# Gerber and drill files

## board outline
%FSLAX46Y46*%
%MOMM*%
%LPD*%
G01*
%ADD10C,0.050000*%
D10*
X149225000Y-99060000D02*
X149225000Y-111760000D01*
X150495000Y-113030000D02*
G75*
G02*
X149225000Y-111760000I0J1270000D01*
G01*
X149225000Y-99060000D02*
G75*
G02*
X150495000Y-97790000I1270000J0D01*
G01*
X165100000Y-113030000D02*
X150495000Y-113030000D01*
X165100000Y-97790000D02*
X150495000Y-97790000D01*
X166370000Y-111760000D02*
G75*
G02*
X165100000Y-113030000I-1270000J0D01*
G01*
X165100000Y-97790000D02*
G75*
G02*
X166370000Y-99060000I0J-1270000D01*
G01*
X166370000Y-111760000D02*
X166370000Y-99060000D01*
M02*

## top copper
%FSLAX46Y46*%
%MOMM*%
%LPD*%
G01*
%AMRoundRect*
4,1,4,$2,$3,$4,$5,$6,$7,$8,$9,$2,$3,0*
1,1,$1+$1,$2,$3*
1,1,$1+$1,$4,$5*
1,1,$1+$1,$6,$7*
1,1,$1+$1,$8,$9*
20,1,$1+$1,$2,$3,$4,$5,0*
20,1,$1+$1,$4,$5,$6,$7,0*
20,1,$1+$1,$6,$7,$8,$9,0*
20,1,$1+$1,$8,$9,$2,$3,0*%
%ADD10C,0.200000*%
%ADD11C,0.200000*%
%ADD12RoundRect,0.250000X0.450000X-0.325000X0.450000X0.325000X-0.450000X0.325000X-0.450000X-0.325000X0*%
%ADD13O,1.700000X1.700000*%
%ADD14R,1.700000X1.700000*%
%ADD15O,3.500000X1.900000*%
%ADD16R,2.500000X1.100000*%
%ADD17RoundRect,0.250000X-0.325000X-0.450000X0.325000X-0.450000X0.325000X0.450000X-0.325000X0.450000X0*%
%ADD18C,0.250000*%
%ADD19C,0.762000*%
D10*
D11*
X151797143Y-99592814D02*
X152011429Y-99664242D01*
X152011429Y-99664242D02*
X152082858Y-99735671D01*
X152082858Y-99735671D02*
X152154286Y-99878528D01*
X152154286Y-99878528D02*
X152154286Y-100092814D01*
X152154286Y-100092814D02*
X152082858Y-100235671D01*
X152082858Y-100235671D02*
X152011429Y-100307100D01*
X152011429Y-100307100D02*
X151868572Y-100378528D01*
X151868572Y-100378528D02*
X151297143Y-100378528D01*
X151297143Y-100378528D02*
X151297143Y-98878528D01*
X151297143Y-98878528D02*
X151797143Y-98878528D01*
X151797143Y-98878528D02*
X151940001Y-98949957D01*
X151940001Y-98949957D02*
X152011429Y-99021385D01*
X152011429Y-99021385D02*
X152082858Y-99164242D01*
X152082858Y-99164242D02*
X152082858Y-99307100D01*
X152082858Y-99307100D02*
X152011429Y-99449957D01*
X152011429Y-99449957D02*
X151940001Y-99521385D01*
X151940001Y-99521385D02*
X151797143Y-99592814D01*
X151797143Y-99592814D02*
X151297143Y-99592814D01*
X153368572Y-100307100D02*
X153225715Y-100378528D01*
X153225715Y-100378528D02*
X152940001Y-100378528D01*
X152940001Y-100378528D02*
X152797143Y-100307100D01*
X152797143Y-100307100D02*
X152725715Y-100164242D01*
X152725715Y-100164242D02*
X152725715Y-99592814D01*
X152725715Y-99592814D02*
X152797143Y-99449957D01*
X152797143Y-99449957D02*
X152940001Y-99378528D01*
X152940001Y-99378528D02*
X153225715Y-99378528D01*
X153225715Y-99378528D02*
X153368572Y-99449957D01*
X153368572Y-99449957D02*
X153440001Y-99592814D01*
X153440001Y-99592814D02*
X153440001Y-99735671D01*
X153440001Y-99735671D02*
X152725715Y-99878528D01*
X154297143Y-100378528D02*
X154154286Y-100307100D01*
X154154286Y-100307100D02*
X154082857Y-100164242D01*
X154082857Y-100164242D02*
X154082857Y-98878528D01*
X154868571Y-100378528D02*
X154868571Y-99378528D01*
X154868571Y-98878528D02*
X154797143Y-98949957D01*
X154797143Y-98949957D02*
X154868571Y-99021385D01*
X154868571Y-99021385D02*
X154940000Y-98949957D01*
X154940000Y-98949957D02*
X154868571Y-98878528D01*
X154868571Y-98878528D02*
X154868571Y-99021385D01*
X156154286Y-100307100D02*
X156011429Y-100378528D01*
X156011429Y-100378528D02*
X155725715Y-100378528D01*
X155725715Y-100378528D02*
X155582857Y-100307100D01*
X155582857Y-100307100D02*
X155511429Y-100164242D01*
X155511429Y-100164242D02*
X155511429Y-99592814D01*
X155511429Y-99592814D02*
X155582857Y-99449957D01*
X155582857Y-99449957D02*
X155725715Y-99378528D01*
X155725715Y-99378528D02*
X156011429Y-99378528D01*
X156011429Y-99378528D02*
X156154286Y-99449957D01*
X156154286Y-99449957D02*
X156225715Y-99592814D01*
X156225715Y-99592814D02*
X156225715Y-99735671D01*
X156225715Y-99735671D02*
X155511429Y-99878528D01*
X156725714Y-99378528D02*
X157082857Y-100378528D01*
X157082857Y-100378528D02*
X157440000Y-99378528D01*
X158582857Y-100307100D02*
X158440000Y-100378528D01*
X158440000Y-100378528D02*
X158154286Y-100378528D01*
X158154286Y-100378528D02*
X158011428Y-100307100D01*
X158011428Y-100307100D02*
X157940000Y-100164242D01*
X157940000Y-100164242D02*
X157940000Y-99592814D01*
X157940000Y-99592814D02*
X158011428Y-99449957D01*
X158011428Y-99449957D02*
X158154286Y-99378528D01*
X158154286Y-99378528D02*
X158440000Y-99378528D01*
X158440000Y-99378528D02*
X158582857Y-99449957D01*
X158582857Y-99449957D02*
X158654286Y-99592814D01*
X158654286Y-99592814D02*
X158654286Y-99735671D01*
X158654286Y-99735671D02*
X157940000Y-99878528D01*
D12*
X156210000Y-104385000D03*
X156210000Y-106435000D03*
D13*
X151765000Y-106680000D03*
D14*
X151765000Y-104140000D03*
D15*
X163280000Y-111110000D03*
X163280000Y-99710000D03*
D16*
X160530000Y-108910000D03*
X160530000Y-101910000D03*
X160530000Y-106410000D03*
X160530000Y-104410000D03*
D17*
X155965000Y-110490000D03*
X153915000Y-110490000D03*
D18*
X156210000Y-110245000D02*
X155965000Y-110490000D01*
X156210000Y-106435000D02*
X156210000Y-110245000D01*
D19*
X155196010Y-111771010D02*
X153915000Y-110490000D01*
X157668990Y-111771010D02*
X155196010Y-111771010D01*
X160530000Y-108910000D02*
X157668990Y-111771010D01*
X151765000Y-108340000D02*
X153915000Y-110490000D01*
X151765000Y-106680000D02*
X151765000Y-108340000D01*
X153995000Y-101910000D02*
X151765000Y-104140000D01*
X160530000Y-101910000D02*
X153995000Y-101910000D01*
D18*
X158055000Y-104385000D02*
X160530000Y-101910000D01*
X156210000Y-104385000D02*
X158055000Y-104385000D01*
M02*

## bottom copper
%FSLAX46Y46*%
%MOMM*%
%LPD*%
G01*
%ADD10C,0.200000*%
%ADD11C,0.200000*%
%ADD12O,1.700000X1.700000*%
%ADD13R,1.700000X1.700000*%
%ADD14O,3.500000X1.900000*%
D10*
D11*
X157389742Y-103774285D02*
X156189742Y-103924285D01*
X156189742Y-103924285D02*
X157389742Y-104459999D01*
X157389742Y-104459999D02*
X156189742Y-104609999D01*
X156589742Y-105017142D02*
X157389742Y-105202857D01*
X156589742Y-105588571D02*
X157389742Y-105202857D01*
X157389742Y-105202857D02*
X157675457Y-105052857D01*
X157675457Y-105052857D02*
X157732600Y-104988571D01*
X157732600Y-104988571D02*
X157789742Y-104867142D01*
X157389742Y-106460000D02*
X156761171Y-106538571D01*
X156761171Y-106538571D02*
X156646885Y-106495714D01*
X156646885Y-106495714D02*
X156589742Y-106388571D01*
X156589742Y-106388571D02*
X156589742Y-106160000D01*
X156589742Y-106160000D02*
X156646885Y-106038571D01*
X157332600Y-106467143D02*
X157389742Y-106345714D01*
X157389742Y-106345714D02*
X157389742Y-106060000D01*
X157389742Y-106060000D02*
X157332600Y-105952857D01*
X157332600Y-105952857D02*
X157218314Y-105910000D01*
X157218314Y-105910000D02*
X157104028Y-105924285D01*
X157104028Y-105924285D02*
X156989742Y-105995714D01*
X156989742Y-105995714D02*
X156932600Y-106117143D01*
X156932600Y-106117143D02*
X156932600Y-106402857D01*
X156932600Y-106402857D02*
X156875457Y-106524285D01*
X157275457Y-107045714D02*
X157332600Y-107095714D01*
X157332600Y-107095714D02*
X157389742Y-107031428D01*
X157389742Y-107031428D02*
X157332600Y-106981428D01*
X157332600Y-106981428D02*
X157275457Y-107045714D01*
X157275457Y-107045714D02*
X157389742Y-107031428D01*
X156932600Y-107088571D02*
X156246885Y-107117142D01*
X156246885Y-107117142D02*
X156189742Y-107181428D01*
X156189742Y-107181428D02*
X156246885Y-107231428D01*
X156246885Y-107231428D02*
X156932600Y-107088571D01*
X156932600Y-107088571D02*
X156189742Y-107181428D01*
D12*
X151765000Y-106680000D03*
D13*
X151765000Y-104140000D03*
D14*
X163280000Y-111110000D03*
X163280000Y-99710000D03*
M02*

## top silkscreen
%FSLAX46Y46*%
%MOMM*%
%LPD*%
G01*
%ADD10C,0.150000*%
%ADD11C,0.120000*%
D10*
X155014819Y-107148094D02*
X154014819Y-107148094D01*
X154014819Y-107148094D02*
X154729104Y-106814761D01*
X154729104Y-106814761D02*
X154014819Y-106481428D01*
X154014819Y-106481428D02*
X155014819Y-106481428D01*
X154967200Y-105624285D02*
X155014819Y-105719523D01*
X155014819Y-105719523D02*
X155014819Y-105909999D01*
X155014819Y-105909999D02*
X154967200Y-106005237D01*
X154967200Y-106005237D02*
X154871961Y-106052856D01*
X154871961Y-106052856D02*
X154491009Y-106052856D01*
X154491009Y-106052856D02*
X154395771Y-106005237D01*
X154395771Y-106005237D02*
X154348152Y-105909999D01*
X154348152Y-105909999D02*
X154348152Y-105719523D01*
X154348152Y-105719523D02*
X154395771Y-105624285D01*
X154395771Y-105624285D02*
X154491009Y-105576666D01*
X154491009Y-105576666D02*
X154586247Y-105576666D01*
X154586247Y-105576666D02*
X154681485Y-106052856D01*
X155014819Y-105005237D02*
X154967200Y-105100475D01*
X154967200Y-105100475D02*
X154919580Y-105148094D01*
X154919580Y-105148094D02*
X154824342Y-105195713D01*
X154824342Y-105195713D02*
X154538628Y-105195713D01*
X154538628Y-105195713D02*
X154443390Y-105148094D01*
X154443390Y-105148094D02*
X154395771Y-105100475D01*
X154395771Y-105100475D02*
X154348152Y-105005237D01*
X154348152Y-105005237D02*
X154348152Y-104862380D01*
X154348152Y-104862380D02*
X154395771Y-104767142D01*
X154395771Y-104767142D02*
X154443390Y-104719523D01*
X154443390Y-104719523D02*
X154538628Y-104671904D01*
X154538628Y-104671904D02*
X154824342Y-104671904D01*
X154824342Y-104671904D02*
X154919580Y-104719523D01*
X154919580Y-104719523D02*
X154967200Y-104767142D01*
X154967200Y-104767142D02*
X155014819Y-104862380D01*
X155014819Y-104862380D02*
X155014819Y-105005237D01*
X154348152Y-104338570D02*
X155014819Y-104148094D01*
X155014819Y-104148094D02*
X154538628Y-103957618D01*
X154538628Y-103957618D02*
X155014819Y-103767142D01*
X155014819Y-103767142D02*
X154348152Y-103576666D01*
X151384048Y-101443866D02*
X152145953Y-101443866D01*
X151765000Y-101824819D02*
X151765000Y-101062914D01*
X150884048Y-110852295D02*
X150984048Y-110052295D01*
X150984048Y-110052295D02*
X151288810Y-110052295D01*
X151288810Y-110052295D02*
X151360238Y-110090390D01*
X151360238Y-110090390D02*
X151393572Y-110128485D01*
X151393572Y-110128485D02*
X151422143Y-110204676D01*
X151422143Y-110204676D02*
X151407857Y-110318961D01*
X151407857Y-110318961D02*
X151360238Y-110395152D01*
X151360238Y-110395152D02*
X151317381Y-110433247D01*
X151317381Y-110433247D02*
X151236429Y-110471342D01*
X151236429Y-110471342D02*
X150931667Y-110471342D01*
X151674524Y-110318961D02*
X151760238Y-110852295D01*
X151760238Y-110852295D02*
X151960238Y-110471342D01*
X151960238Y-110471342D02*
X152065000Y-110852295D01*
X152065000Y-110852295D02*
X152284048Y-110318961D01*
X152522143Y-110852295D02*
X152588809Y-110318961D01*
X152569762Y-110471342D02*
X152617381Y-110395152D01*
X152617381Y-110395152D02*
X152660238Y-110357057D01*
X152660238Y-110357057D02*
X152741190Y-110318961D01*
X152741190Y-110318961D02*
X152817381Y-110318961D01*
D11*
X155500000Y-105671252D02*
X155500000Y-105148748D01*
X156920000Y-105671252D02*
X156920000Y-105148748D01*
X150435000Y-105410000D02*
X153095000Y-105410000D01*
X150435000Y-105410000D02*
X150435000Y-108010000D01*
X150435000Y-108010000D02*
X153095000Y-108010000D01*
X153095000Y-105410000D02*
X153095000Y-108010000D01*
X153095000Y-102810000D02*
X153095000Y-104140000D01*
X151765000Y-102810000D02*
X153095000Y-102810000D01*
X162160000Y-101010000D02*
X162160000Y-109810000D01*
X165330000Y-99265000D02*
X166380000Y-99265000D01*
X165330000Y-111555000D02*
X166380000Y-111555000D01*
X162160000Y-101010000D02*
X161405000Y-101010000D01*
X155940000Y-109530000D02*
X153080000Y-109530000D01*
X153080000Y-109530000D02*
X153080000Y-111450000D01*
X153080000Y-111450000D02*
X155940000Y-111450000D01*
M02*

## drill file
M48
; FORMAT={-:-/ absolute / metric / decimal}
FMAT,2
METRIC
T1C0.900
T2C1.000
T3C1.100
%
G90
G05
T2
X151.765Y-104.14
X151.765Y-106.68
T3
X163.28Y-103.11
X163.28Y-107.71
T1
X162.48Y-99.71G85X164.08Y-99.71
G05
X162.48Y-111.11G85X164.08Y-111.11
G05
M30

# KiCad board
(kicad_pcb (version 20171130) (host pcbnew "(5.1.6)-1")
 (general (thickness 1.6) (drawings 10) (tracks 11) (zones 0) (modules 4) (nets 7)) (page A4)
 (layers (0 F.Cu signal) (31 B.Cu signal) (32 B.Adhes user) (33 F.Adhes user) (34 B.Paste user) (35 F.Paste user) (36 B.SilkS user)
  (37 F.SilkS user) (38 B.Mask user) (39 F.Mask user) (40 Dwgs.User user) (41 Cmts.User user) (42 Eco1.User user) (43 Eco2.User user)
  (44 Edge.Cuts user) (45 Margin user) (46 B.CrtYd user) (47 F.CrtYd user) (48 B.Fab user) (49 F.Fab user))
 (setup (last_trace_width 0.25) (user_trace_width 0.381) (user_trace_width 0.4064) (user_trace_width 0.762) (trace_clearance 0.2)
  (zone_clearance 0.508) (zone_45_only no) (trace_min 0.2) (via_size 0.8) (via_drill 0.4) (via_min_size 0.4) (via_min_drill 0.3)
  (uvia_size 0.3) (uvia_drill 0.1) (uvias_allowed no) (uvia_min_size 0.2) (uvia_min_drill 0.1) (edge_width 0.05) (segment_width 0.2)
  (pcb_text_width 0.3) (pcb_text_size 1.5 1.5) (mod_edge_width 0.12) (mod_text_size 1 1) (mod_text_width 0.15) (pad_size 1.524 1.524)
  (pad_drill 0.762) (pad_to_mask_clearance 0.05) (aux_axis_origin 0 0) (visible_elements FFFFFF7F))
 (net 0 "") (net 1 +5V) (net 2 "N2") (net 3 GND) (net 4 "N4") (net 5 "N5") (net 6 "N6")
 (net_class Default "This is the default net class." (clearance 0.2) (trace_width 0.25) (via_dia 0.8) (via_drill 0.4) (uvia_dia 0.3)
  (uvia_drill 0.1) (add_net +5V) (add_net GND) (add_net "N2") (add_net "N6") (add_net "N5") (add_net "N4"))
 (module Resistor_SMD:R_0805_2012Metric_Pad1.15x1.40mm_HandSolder (layer F.Cu) (at 156.21 105.41 90)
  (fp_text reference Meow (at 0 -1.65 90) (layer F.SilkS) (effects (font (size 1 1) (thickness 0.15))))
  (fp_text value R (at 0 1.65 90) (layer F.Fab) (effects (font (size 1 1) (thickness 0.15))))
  (fp_line (start -0.261252 -0.71) (end 0.261252 -0.71) (layer F.SilkS) (width 0.12))
  (fp_line (start -0.261252 0.71) (end 0.261252 0.71) (layer F.SilkS) (width 0.12))
  (pad 2 smd roundrect (at 1.025 0 90) (size 1.15 1.4) (layers F.Cu F.Paste F.Mask) (roundrect_rratio 0.217391) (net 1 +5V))
  (pad 1 smd roundrect (at -1.025 0 90) (size 1.15 1.4) (layers F.Cu F.Paste F.Mask) (roundrect_rratio 0.217391) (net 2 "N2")))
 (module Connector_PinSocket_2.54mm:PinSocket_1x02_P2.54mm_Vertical (layer F.Cu) (at 151.765 104.14)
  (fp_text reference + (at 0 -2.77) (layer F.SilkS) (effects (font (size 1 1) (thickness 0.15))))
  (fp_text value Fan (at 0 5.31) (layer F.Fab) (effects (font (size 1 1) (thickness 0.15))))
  (fp_line (start -1.33 1.27) (end 1.33 1.27) (layer F.SilkS) (width 0.12))
  (fp_line (start -1.33 1.27) (end -1.33 3.87) (layer F.SilkS) (width 0.12))
  (fp_line (start -1.33 3.87) (end 1.33 3.87) (layer F.SilkS) (width 0.12))
  (fp_line (start 1.33 1.27) (end 1.33 3.87) (layer F.SilkS) (width 0.12))
  (fp_line (start 1.33 -1.33) (end 1.33 0) (layer F.SilkS) (width 0.12))
  (fp_line (start 0 -1.33) (end 1.33 -1.33) (layer F.SilkS) (width 0.12))
  (pad 2 thru_hole oval (at 0 2.54) (size 1.7 1.7) (drill 1) (layers *.Cu *.Mask) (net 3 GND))
  (pad 1 thru_hole rect (at 0 0) (size 1.7 1.7) (drill 1) (layers *.Cu *.Mask) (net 1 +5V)))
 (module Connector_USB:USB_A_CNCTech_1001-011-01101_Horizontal (layer F.Cu) (at 170.18 105.41)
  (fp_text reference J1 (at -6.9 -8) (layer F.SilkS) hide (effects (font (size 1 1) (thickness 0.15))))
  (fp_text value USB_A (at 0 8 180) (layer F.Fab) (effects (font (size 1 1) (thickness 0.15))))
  (fp_line (start -8.02 -4.4) (end -8.02 4.4) (layer F.SilkS) (width 0.12))
  (fp_line (start -4.85 -6.145) (end -3.8 -6.145) (layer F.SilkS) (width 0.12))
  (fp_line (start -4.85 6.145) (end -3.8 6.145) (layer F.SilkS) (width 0.12))
  (fp_line (start -8.02 -4.4) (end -8.775 -4.4) (layer F.SilkS) (width 0.12))
  (pad "" np_thru_hole circle (at -6.9 2.3) (size 1.1 1.1) (drill 1.1) (layers *.Cu *.Mask))
  (pad "" np_thru_hole circle (at -6.9 -2.3) (size 1.1 1.1) (drill 1.1) (layers *.Cu *.Mask))
  (pad 5 thru_hole oval (at -6.9 5.7) (size 3.5 1.9) (drill oval 2.5 0.9) (layers *.Cu *.Mask) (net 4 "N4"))
  (pad 5 thru_hole oval (at -6.9 -5.7) (size 3.5 1.9) (drill oval 2.5 0.9) (layers *.Cu *.Mask) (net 4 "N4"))
  (pad 4 smd rect (at -9.65 3.5) (size 2.5 1.1) (layers F.Cu F.Paste F.Mask) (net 3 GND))
  (pad 1 smd rect (at -9.65 -3.5) (size 2.5 1.1) (layers F.Cu F.Paste F.Mask) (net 1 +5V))
  (pad 3 smd rect (at -9.65 1) (size 2.5 1.1) (layers F.Cu F.Paste F.Mask) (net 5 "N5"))
  (pad 2 smd rect (at -9.65 -1) (size 2.5 1.1) (layers F.Cu F.Paste F.Mask) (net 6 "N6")))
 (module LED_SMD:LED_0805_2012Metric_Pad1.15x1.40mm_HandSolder (layer F.Cu) (at 154.94 110.49)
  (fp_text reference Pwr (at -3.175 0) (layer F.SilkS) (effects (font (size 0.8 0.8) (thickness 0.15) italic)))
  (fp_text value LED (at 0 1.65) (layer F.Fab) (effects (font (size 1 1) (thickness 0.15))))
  (fp_line (start 1 -0.96) (end -1.86 -0.96) (layer F.SilkS) (width 0.12))
  (fp_line (start -1.86 -0.96) (end -1.86 0.96) (layer F.SilkS) (width 0.12))
  (fp_line (start -1.86 0.96) (end 1 0.96) (layer F.SilkS) (width 0.12))
  (pad 2 smd roundrect (at 1.025 0) (size 1.15 1.4) (layers F.Cu F.Paste F.Mask) (roundrect_rratio 0.217391) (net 2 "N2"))
  (pad 1 smd roundrect (at -1.025 0) (size 1.15 1.4) (layers F.Cu F.Paste F.Mask) (roundrect_rratio 0.217391) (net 3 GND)))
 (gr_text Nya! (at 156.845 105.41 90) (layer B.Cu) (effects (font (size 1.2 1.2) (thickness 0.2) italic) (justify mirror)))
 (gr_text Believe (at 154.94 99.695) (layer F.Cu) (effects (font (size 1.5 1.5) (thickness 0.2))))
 (gr_line (start 149.225 99.06) (end 149.225 111.76) (layer Edge.Cuts) (width 0.05))
 (gr_arc (start 150.495 111.76) (end 149.225 111.76) (angle -90) (layer Edge.Cuts) (width 0.05))
 (gr_arc (start 150.495 99.06) (end 150.495 97.79) (angle -90) (layer Edge.Cuts) (width 0.05))
 (gr_line (start 165.1 113.03) (end 150.495 113.03) (layer Edge.Cuts) (width 0.05))
 (gr_line (start 165.1 97.79) (end 150.495 97.79) (layer Edge.Cuts) (width 0.05))
 (gr_arc (start 165.1 111.76) (end 165.1 113.03) (angle -90) (layer Edge.Cuts) (width 0.05))
 (gr_arc (start 165.1 99.06) (end 166.37 99.06) (angle -90) (layer Edge.Cuts) (width 0.05))
 (gr_line (start 166.37 111.76) (end 166.37 99.06) (layer Edge.Cuts) (width 0.05))
 (segment (start 156.21 110.245) (end 155.965 110.49) (width 0.25) (layer F.Cu) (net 2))
 (segment (start 156.21 106.435) (end 156.21 110.245) (width 0.25) (layer F.Cu) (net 2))
 (segment (start 155.19601 111.77101) (end 153.915 110.49) (width 0.762) (layer F.Cu) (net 3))
 (segment (start 157.66899 111.77101) (end 155.19601 111.77101) (width 0.762) (layer F.Cu) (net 3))
 (segment (start 160.53 108.91) (end 157.66899 111.77101) (width 0.762) (layer F.Cu) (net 3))
 (segment (start 151.765 108.34) (end 153.915 110.49) (width 0.762) (layer F.Cu) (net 3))
 (segment (start 151.765 106.68) (end 151.765 108.34) (width 0.762) (layer F.Cu) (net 3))
 (segment (start 153.995 101.91) (end 151.765 104.14) (width 0.762) (layer F.Cu) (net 1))
 (segment (start 160.53 101.91) (end 153.995 101.91) (width 0.762) (layer F.Cu) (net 1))
 (segment (start 158.055 104.385) (end 160.53 101.91) (width 0.25) (layer F.Cu) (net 1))
 (segment (start 156.21 104.385) (end 158.055 104.385) (width 0.25) (layer F.Cu) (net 1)))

